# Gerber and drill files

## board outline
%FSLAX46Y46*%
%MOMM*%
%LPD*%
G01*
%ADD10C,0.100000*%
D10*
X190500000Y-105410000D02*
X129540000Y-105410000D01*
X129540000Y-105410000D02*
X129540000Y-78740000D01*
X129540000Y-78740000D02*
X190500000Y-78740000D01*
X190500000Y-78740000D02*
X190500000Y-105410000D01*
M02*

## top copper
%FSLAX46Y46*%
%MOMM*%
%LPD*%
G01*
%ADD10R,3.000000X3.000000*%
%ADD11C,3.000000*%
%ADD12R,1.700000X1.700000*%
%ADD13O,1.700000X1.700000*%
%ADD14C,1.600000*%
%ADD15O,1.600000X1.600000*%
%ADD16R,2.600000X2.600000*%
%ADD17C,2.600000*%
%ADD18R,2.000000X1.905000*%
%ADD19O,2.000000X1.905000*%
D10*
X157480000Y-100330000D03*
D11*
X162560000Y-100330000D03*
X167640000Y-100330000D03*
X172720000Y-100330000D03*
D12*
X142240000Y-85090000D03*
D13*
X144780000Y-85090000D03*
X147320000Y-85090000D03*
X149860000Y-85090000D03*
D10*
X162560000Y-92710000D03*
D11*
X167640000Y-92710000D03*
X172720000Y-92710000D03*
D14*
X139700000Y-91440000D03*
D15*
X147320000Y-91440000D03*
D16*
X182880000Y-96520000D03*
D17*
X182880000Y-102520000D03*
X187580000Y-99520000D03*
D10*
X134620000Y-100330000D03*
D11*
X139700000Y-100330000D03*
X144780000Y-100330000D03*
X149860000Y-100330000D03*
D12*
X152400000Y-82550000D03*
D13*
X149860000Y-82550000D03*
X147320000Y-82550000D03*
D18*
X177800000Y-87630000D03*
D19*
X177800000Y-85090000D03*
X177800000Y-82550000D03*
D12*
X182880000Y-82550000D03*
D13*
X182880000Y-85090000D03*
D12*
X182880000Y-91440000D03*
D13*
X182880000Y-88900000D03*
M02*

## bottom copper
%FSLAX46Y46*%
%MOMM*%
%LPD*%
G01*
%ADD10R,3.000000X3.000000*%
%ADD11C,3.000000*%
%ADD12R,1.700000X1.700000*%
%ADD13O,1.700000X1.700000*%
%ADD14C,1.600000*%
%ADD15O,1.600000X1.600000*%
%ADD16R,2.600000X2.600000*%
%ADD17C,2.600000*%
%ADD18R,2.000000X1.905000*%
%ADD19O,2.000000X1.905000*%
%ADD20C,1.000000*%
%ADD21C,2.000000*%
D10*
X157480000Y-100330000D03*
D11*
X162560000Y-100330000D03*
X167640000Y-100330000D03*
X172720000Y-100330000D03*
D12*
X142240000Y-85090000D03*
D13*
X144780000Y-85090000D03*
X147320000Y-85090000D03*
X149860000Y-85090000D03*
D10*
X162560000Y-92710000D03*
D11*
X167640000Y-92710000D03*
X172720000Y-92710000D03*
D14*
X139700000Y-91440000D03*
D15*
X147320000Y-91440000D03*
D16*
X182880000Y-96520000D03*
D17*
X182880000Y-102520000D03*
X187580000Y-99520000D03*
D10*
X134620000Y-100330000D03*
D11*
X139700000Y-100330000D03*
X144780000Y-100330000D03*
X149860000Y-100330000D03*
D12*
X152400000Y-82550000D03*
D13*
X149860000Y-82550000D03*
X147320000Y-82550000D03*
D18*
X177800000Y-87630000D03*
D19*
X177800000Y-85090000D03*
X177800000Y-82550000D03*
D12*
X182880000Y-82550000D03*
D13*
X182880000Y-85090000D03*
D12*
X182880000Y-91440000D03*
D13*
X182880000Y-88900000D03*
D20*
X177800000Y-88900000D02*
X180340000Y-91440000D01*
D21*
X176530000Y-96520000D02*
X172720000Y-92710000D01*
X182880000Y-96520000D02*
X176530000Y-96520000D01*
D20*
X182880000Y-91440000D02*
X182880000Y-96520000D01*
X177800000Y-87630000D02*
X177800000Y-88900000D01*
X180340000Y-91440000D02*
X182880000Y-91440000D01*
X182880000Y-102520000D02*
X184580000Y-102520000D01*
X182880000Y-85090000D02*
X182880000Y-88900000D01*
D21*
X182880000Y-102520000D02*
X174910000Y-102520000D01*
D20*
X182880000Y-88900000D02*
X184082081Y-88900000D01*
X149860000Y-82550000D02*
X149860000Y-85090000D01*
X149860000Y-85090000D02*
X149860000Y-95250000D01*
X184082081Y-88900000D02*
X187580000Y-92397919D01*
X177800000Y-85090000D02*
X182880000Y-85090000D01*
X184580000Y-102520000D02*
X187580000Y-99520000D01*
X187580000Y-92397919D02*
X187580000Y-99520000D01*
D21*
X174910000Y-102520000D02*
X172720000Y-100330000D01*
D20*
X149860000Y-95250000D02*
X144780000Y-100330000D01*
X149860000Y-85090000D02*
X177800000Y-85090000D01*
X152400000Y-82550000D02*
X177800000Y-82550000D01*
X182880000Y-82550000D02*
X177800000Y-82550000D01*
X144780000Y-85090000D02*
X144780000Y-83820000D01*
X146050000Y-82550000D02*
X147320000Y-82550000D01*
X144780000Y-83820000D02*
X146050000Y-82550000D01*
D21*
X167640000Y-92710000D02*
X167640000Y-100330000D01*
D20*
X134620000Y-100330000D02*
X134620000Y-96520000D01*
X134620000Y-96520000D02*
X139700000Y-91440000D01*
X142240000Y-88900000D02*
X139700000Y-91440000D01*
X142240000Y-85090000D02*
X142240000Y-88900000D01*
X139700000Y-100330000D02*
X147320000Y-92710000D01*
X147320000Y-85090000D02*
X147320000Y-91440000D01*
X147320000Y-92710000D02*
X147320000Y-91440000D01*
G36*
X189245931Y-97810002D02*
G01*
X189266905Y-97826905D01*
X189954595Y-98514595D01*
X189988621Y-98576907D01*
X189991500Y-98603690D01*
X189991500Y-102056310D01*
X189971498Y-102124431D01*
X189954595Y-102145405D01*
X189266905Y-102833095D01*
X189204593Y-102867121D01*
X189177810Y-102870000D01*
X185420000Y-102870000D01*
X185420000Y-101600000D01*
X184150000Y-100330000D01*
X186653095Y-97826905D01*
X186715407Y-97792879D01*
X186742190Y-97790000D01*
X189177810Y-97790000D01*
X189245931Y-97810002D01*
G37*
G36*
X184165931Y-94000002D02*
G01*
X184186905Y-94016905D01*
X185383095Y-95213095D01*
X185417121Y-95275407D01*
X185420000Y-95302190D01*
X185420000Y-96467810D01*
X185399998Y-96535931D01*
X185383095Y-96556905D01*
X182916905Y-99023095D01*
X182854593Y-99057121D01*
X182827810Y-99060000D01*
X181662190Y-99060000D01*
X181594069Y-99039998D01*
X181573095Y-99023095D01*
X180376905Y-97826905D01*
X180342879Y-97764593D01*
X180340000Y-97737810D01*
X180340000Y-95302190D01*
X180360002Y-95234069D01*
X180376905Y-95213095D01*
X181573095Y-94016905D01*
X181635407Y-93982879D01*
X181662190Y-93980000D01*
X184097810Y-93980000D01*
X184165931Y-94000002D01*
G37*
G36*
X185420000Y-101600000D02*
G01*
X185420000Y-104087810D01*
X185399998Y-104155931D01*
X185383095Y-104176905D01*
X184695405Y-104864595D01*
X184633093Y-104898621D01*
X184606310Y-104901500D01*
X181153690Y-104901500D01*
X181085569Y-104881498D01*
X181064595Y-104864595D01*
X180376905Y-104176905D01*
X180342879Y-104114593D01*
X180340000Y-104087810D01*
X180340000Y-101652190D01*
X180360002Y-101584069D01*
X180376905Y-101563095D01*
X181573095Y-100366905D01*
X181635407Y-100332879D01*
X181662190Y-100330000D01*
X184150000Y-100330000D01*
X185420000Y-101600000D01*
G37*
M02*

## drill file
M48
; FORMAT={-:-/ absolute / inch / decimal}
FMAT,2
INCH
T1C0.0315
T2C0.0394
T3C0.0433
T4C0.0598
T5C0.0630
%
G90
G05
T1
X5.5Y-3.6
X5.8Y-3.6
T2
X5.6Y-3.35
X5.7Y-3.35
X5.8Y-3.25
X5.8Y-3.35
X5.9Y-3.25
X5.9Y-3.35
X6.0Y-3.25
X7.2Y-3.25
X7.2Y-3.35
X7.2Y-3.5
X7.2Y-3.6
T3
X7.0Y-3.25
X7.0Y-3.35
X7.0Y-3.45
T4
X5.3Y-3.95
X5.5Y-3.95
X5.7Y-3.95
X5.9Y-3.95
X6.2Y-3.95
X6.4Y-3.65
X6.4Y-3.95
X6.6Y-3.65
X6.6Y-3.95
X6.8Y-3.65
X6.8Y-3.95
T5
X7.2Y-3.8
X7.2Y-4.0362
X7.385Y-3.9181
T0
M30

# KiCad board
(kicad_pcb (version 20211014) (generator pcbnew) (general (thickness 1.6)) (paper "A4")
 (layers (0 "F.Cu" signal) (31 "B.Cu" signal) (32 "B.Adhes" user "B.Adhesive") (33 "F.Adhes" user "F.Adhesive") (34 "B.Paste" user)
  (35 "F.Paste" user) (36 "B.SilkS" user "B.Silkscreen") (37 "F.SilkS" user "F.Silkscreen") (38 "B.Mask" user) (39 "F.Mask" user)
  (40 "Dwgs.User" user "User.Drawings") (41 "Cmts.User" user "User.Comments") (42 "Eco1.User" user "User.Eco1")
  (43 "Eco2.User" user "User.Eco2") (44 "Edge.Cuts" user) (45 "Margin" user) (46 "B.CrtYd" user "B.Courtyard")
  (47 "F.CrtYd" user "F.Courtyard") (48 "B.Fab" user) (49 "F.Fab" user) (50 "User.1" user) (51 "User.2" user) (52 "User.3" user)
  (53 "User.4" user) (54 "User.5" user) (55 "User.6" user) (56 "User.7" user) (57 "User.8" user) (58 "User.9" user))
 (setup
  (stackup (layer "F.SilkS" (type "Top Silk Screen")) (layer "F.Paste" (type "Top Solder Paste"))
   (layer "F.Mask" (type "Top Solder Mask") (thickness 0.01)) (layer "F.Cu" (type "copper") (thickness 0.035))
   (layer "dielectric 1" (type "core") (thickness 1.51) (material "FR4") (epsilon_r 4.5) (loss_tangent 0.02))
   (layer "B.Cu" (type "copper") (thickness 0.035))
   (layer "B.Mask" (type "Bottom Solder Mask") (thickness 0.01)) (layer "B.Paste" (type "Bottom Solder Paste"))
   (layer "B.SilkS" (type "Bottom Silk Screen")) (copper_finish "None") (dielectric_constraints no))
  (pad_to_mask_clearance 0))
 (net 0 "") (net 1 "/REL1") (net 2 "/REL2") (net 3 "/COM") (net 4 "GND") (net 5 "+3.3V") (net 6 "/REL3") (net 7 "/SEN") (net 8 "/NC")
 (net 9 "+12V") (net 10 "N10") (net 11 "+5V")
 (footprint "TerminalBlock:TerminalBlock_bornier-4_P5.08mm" (layer "F.Cu") (at 157.48 100.33)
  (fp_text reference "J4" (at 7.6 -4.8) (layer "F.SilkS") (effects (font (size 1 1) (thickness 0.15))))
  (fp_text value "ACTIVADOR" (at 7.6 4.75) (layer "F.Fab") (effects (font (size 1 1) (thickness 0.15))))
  (pad "1" thru_hole rect (at 0 0) (size 3 3) (drill 1.52) (layers *.Cu *.Mask) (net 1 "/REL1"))
  (pad "2" thru_hole circle (at 5.08 0) (size 3 3) (drill 1.52) (layers *.Cu *.Mask) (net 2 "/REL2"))
  (pad "3" thru_hole circle (at 10.16 0) (size 3 3) (drill 1.52) (layers *.Cu *.Mask) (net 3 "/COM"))
  (pad "4" thru_hole circle (at 15.24 0) (size 3 3) (drill 1.52) (layers *.Cu *.Mask) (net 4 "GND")))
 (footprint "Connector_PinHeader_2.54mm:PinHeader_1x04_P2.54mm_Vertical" (layer "F.Cu") (at 142.24 85.09 90)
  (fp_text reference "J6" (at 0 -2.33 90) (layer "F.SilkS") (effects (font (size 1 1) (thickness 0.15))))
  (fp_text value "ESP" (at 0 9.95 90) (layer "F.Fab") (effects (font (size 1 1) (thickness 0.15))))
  (pad "1" thru_hole rect (at 0 0 90) (size 1.7 1.7) (drill 1) (layers *.Cu *.Mask) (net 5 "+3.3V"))
  (pad "2" thru_hole oval (at 0 2.54 90) (size 1.7 1.7) (drill 1) (layers *.Cu *.Mask) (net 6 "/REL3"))
  (pad "3" thru_hole oval (at 0 5.08 90) (size 1.7 1.7) (drill 1) (layers *.Cu *.Mask) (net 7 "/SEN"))
  (pad "4" thru_hole oval (at 0 7.62 90) (size 1.7 1.7) (drill 1) (layers *.Cu *.Mask) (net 4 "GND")))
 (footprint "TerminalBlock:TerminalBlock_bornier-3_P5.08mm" (layer "F.Cu") (at 162.56 92.71)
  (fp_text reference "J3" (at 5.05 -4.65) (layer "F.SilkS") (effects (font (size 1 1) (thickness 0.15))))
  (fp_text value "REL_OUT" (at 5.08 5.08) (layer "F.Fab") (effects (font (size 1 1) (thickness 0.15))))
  (pad "1" thru_hole rect (at 0 0) (size 3 3) (drill 1.52) (layers *.Cu *.Mask) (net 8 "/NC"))
  (pad "2" thru_hole circle (at 5.08 0) (size 3 3) (drill 1.52) (layers *.Cu *.Mask) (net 3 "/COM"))
  (pad "3" thru_hole circle (at 10.16 0) (size 3 3) (drill 1.52) (layers *.Cu *.Mask) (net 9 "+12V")))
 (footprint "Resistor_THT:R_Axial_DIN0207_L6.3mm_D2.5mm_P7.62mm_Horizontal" (layer "F.Cu") (at 139.7 91.44)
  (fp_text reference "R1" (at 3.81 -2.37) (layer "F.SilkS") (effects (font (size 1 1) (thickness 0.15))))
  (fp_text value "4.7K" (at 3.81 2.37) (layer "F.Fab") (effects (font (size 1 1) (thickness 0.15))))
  (pad "1" thru_hole circle (at 0 0) (size 1.6 1.6) (drill 0.8) (layers *.Cu *.Mask) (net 5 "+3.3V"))
  (pad "2" thru_hole oval (at 7.62 0) (size 1.6 1.6) (drill 0.8) (layers *.Cu *.Mask) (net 7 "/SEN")))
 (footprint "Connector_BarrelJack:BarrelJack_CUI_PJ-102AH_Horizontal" (layer "F.Cu") (at 182.88 96.52)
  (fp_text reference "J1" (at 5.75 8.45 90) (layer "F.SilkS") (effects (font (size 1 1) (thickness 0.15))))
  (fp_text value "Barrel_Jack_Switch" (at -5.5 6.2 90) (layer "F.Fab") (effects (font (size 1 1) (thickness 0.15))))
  (pad "1" thru_hole rect (at 0 0) (size 2.6 2.6) (drill 1.6) (layers *.Cu *.Mask) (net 9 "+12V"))
  (pad "2" thru_hole circle (at 0 6) (size 2.6 2.6) (drill 1.6) (layers *.Cu *.Mask) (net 4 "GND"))
  (pad "3" thru_hole circle (at 4.7 3) (size 2.6 2.6) (drill 1.6) (layers *.Cu *.Mask) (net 4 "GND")))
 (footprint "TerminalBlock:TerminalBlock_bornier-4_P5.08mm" (layer "F.Cu") (at 134.62 100.33)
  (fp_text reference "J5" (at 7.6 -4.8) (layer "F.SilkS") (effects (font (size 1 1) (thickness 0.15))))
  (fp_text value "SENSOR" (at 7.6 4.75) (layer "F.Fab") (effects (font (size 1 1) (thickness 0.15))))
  (pad "1" thru_hole rect (at 0 0) (size 3 3) (drill 1.52) (layers *.Cu *.Mask) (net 5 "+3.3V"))
  (pad "2" thru_hole circle (at 5.08 0) (size 3 3) (drill 1.52) (layers *.Cu *.Mask) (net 7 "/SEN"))
  (pad "3" thru_hole circle (at 10.16 0) (size 3 3) (drill 1.52) (layers *.Cu *.Mask) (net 4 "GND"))
  (pad "4" thru_hole circle (at 15.24 0) (size 3 3) (drill 1.52) (layers *.Cu *.Mask) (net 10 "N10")))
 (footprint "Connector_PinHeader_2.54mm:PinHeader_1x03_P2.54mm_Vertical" (layer "F.Cu") (at 152.4 82.55 -90)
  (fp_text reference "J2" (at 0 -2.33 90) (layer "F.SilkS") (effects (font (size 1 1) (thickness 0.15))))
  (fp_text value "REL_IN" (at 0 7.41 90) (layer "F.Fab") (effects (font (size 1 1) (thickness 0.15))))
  (pad "1" thru_hole rect (at 0 0 270) (size 1.7 1.7) (drill 1) (layers *.Cu *.Mask) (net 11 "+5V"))
  (pad "2" thru_hole oval (at 0 2.54 270) (size 1.7 1.7) (drill 1) (layers *.Cu *.Mask) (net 4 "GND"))
  (pad "3" thru_hole oval (at 0 5.08 270) (size 1.7 1.7) (drill 1) (layers *.Cu *.Mask) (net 6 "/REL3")))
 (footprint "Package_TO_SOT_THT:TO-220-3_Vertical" (layer "F.Cu") (at 177.8 87.63 90)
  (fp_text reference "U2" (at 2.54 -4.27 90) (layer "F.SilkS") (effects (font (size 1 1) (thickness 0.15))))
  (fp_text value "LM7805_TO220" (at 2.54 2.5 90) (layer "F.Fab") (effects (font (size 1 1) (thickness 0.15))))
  (pad "1" thru_hole rect (at 0 0 90) (size 1.905 2) (drill 1.1) (layers *.Cu *.Mask) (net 9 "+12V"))
  (pad "2" thru_hole oval (at 2.54 0 90) (size 1.905 2) (drill 1.1) (layers *.Cu *.Mask) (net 4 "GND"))
  (pad "3" thru_hole oval (at 5.08 0 90) (size 1.905 2) (drill 1.1) (layers *.Cu *.Mask) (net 11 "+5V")))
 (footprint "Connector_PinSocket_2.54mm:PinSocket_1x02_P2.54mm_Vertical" (layer "F.Cu") (at 182.88 82.55)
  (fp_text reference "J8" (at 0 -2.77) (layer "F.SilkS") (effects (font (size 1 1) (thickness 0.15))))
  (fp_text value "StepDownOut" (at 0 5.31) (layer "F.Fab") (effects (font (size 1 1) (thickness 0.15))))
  (pad "1" thru_hole rect (at 0 0) (size 1.7 1.7) (drill 1) (layers *.Cu *.Mask) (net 11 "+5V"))
  (pad "2" thru_hole oval (at 0 2.54) (size 1.7 1.7) (drill 1) (layers *.Cu *.Mask) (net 4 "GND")))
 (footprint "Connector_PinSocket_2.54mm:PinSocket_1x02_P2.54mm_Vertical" (layer "F.Cu") (at 182.88 91.44 180)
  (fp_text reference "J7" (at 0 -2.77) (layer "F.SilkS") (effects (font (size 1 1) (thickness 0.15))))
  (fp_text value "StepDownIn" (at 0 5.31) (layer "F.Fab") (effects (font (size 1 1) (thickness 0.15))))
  (pad "1" thru_hole rect (at 0 0 180) (size 1.7 1.7) (drill 1) (layers *.Cu *.Mask) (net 9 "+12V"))
  (pad "2" thru_hole oval (at 0 2.54 180) (size 1.7 1.7) (drill 1) (layers *.Cu *.Mask) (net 4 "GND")))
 (gr_rect (start 190.5 105.41) (end 129.54 78.74) (layer "Edge.Cuts") (width 0.1) (fill none))
 (segment (start 177.8 88.9) (end 180.34 91.44) (width 1) (layer "B.Cu") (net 9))
 (segment (start 176.53 96.52) (end 172.72 92.71) (width 2) (layer "B.Cu") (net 9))
 (segment (start 182.88 96.52) (end 176.53 96.52) (width 2) (layer "B.Cu") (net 9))
 (segment (start 182.88 91.44) (end 182.88 96.52) (width 1) (layer "B.Cu") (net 9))
 (segment (start 177.8 87.63) (end 177.8 88.9) (width 1) (layer "B.Cu") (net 9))
 (segment (start 180.34 91.44) (end 182.88 91.44) (width 1) (layer "B.Cu") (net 9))
 (segment (start 182.88 102.52) (end 184.58 102.52) (width 1) (layer "B.Cu") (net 4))
 (segment (start 182.88 85.09) (end 182.88 88.9) (width 1) (layer "B.Cu") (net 4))
 (segment (start 182.88 102.52) (end 174.91 102.52) (width 2) (layer "B.Cu") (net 4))
 (segment (start 182.88 88.9) (end 184.082081 88.9) (width 1) (layer "B.Cu") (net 4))
 (segment (start 149.86 82.55) (end 149.86 85.09) (width 1) (layer "B.Cu") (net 4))
 (segment (start 149.86 85.09) (end 149.86 95.25) (width 1) (layer "B.Cu") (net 4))
 (segment (start 184.082081 88.9) (end 187.58 92.397919) (width 1) (layer "B.Cu") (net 4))
 (segment (start 177.8 85.09) (end 182.88 85.09) (width 1) (layer "B.Cu") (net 4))
 (segment (start 184.58 102.52) (end 187.58 99.52) (width 1) (layer "B.Cu") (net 4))
 (segment (start 187.58 92.397919) (end 187.58 99.52) (width 1) (layer "B.Cu") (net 4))
 (segment (start 174.91 102.52) (end 172.72 100.33) (width 2) (layer "B.Cu") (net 4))
 (segment (start 149.86 95.25) (end 144.78 100.33) (width 1) (layer "B.Cu") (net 4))
 (segment (start 149.86 85.09) (end 177.8 85.09) (width 1) (layer "B.Cu") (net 4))
 (segment (start 152.4 82.55) (end 177.8 82.55) (width 1) (layer "B.Cu") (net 11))
 (segment (start 182.88 82.55) (end 177.8 82.55) (width 1) (layer "B.Cu") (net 11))
 (segment (start 144.78 85.09) (end 144.78 83.82) (width 1) (layer "B.Cu") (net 6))
 (segment (start 146.05 82.55) (end 147.32 82.55) (width 1) (layer "B.Cu") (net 6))
 (segment (start 144.78 83.82) (end 146.05 82.55) (width 1) (layer "B.Cu") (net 6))
 (segment (start 167.64 92.71) (end 167.64 100.33) (width 2) (layer "B.Cu") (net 3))
 (segment (start 134.62 100.33) (end 134.62 96.52) (width 1) (layer "B.Cu") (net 5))
 (segment (start 134.62 96.52) (end 139.7 91.44) (width 1) (layer "B.Cu") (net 5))
 (segment (start 142.24 88.9) (end 139.7 91.44) (width 1) (layer "B.Cu") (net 5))
 (segment (start 142.24 85.09) (end 142.24 88.9) (width 1) (layer "B.Cu") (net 5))
 (segment (start 139.7 100.33) (end 147.32 92.71) (width 1) (layer "B.Cu") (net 7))
 (segment (start 147.32 85.09) (end 147.32 91.44) (width 1) (layer "B.Cu") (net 7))
 (segment (start 147.32 92.71) (end 147.32 91.44) (width 1) (layer "B.Cu") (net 7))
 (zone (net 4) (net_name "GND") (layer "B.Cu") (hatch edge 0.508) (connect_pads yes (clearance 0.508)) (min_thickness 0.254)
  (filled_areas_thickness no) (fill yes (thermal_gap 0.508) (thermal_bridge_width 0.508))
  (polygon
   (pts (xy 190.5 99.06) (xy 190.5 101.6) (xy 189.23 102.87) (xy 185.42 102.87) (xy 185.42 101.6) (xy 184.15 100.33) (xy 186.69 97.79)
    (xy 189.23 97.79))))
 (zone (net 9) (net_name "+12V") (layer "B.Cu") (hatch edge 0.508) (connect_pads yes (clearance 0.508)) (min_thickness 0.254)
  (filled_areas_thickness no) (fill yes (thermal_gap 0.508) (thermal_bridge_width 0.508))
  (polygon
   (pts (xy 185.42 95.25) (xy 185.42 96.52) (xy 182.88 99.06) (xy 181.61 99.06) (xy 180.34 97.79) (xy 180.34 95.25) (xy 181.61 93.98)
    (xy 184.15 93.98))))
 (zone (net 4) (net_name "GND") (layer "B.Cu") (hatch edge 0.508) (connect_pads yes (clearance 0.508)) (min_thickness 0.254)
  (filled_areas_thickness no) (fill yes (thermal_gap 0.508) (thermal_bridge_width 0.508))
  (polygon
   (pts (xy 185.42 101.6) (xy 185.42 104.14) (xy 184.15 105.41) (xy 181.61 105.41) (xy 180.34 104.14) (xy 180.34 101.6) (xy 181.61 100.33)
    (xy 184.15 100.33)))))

